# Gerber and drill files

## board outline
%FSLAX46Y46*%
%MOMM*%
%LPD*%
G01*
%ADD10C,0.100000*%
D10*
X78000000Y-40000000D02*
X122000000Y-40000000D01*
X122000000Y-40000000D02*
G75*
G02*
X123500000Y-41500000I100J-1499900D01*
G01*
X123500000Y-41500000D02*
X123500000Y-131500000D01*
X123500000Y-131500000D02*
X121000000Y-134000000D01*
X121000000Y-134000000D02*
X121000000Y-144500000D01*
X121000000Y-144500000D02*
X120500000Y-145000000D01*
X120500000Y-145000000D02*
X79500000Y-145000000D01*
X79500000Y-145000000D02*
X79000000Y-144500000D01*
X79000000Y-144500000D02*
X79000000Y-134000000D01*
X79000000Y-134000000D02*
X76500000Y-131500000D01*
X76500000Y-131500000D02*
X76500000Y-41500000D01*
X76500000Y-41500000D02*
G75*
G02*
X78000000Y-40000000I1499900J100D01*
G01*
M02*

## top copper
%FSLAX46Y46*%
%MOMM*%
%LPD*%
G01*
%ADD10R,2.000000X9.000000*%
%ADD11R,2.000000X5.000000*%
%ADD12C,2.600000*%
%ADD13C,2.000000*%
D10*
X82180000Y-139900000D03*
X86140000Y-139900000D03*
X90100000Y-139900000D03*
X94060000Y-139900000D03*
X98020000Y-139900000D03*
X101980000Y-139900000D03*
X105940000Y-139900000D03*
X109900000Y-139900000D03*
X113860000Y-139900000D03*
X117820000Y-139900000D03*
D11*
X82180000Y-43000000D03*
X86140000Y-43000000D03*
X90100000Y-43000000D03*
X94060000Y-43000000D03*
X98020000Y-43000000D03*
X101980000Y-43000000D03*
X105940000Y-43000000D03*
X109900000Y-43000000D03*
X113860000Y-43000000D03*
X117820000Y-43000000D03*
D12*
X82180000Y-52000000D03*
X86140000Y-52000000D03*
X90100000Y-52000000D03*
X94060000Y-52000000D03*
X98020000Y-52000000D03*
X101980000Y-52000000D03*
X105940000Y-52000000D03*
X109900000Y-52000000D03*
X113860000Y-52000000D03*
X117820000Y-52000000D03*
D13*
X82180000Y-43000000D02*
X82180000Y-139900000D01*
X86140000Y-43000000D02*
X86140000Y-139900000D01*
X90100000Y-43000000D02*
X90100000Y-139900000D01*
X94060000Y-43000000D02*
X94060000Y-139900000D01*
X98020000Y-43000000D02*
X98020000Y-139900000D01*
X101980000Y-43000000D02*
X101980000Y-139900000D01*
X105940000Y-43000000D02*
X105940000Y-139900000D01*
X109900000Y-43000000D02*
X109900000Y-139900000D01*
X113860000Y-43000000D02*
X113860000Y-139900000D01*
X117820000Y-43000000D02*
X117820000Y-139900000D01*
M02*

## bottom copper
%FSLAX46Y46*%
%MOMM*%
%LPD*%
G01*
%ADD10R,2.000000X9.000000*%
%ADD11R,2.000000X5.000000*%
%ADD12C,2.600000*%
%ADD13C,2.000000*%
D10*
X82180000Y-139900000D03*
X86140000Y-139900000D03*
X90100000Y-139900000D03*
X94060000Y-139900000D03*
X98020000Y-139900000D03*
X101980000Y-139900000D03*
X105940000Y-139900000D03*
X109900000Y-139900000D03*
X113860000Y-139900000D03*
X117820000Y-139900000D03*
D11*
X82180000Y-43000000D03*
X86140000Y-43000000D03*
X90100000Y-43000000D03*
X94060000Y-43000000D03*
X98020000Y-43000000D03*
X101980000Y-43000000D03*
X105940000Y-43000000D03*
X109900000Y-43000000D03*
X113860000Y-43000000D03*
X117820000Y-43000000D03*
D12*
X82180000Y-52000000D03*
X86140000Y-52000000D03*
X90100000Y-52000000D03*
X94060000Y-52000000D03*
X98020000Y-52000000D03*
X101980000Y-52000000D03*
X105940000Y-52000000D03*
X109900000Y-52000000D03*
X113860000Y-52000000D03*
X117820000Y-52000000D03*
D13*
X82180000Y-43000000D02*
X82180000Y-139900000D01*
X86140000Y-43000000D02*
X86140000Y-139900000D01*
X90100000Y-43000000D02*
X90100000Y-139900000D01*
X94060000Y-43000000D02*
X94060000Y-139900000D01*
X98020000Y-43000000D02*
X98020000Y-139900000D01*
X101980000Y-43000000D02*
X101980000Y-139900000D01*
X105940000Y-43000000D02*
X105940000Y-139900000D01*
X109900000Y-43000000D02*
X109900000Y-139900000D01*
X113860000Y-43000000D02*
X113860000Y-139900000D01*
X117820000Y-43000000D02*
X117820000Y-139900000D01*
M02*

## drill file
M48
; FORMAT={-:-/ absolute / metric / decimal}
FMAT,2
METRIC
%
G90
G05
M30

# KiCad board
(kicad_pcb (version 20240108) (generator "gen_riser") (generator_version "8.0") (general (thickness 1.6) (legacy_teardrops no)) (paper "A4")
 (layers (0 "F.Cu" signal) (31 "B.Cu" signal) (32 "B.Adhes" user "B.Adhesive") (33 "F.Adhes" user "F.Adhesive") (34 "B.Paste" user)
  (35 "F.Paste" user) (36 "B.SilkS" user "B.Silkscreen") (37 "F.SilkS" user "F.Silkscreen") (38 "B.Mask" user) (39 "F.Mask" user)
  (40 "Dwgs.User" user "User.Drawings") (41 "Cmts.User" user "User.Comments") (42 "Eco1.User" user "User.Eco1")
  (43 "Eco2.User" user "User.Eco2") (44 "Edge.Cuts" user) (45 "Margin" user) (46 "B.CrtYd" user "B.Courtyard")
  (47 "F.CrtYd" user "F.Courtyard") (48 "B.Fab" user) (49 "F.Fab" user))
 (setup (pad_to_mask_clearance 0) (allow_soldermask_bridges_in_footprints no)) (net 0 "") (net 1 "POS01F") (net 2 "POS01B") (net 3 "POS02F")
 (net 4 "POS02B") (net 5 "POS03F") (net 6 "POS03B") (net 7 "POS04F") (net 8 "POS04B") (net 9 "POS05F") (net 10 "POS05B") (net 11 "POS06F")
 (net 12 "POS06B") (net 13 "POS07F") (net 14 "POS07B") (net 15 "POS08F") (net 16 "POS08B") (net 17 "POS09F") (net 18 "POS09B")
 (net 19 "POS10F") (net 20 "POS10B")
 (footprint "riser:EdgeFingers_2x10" (layer "F.Cu") (at 100 40)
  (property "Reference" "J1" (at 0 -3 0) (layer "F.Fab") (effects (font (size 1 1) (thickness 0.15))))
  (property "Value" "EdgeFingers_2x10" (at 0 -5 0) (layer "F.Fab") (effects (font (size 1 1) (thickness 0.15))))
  (pad "1" smd rect (at -17.82 99.9) (size 2 9) (layers "F.Cu" "F.Mask") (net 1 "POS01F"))
  (pad "1B" smd rect (at -17.82 99.9) (size 2 9) (layers "B.Cu" "B.Mask") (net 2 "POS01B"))
  (pad "2" smd rect (at -13.86 99.9) (size 2 9) (layers "F.Cu" "F.Mask") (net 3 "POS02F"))
  (pad "2B" smd rect (at -13.86 99.9) (size 2 9) (layers "B.Cu" "B.Mask") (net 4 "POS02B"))
  (pad "3" smd rect (at -9.9 99.9) (size 2 9) (layers "F.Cu" "F.Mask") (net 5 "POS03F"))
  (pad "3B" smd rect (at -9.9 99.9) (size 2 9) (layers "B.Cu" "B.Mask") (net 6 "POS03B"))
  (pad "4" smd rect (at -5.94 99.9) (size 2 9) (layers "F.Cu" "F.Mask") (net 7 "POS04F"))
  (pad "4B" smd rect (at -5.94 99.9) (size 2 9) (layers "B.Cu" "B.Mask") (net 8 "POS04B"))
  (pad "5" smd rect (at -1.98 99.9) (size 2 9) (layers "F.Cu" "F.Mask") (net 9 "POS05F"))
  (pad "5B" smd rect (at -1.98 99.9) (size 2 9) (layers "B.Cu" "B.Mask") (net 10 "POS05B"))
  (pad "6" smd rect (at 1.98 99.9) (size 2 9) (layers "F.Cu" "F.Mask") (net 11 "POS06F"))
  (pad "6B" smd rect (at 1.98 99.9) (size 2 9) (layers "B.Cu" "B.Mask") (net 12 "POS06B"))
  (pad "7" smd rect (at 5.94 99.9) (size 2 9) (layers "F.Cu" "F.Mask") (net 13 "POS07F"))
  (pad "7B" smd rect (at 5.94 99.9) (size 2 9) (layers "B.Cu" "B.Mask") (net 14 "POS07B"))
  (pad "8" smd rect (at 9.9 99.9) (size 2 9) (layers "F.Cu" "F.Mask") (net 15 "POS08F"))
  (pad "8B" smd rect (at 9.9 99.9) (size 2 9) (layers "B.Cu" "B.Mask") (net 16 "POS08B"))
  (pad "9" smd rect (at 13.86 99.9) (size 2 9) (layers "F.Cu" "F.Mask") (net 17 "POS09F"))
  (pad "9B" smd rect (at 13.86 99.9) (size 2 9) (layers "B.Cu" "B.Mask") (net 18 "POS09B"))
  (pad "10" smd rect (at 17.82 99.9) (size 2 9) (layers "F.Cu" "F.Mask") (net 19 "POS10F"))
  (pad "10B" smd rect (at 17.82 99.9) (size 2 9) (layers "B.Cu" "B.Mask") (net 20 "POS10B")))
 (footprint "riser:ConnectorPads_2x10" (layer "F.Cu") (at 100 40)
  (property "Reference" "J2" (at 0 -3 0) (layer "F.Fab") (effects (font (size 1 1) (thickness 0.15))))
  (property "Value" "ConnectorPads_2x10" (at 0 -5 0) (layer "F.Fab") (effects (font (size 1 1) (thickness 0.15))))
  (pad "1" smd rect (at -17.82 3) (size 2 5) (layers "F.Cu" "F.Mask") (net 1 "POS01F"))
  (pad "1B" smd rect (at -17.82 3) (size 2 5) (layers "B.Cu" "B.Mask") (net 2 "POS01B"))
  (pad "2" smd rect (at -13.86 3) (size 2 5) (layers "F.Cu" "F.Mask") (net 3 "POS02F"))
  (pad "2B" smd rect (at -13.86 3) (size 2 5) (layers "B.Cu" "B.Mask") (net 4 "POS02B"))
  (pad "3" smd rect (at -9.9 3) (size 2 5) (layers "F.Cu" "F.Mask") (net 5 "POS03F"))
  (pad "3B" smd rect (at -9.9 3) (size 2 5) (layers "B.Cu" "B.Mask") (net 6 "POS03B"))
  (pad "4" smd rect (at -5.94 3) (size 2 5) (layers "F.Cu" "F.Mask") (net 7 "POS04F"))
  (pad "4B" smd rect (at -5.94 3) (size 2 5) (layers "B.Cu" "B.Mask") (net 8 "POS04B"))
  (pad "5" smd rect (at -1.98 3) (size 2 5) (layers "F.Cu" "F.Mask") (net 9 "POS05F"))
  (pad "5B" smd rect (at -1.98 3) (size 2 5) (layers "B.Cu" "B.Mask") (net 10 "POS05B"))
  (pad "6" smd rect (at 1.98 3) (size 2 5) (layers "F.Cu" "F.Mask") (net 11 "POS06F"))
  (pad "6B" smd rect (at 1.98 3) (size 2 5) (layers "B.Cu" "B.Mask") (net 12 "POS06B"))
  (pad "7" smd rect (at 5.94 3) (size 2 5) (layers "F.Cu" "F.Mask") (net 13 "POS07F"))
  (pad "7B" smd rect (at 5.94 3) (size 2 5) (layers "B.Cu" "B.Mask") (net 14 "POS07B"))
  (pad "8" smd rect (at 9.9 3) (size 2 5) (layers "F.Cu" "F.Mask") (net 15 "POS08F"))
  (pad "8B" smd rect (at 9.9 3) (size 2 5) (layers "B.Cu" "B.Mask") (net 16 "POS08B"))
  (pad "9" smd rect (at 13.86 3) (size 2 5) (layers "F.Cu" "F.Mask") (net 17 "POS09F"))
  (pad "9B" smd rect (at 13.86 3) (size 2 5) (layers "B.Cu" "B.Mask") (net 18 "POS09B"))
  (pad "10" smd rect (at 17.82 3) (size 2 5) (layers "F.Cu" "F.Mask") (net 19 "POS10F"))
  (pad "10B" smd rect (at 17.82 3) (size 2 5) (layers "B.Cu" "B.Mask") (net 20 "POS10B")))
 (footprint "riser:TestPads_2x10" (layer "F.Cu") (at 100 40)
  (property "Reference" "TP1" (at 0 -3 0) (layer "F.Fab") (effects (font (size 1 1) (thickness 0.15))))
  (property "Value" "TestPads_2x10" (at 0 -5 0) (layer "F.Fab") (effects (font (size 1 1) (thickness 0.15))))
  (pad "1" smd circle (at -17.82 12) (size 2.6 2.6) (layers "F.Cu" "F.Mask") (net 1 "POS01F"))
  (pad "1B" smd circle (at -17.82 12) (size 2.6 2.6) (layers "B.Cu" "B.Mask") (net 2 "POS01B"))
  (pad "2" smd circle (at -13.86 12) (size 2.6 2.6) (layers "F.Cu" "F.Mask") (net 3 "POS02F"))
  (pad "2B" smd circle (at -13.86 12) (size 2.6 2.6) (layers "B.Cu" "B.Mask") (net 4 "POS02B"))
  (pad "3" smd circle (at -9.9 12) (size 2.6 2.6) (layers "F.Cu" "F.Mask") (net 5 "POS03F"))
  (pad "3B" smd circle (at -9.9 12) (size 2.6 2.6) (layers "B.Cu" "B.Mask") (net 6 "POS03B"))
  (pad "4" smd circle (at -5.94 12) (size 2.6 2.6) (layers "F.Cu" "F.Mask") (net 7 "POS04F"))
  (pad "4B" smd circle (at -5.94 12) (size 2.6 2.6) (layers "B.Cu" "B.Mask") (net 8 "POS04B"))
  (pad "5" smd circle (at -1.98 12) (size 2.6 2.6) (layers "F.Cu" "F.Mask") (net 9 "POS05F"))
  (pad "5B" smd circle (at -1.98 12) (size 2.6 2.6) (layers "B.Cu" "B.Mask") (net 10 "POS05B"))
  (pad "6" smd circle (at 1.98 12) (size 2.6 2.6) (layers "F.Cu" "F.Mask") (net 11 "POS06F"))
  (pad "6B" smd circle (at 1.98 12) (size 2.6 2.6) (layers "B.Cu" "B.Mask") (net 12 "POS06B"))
  (pad "7" smd circle (at 5.94 12) (size 2.6 2.6) (layers "F.Cu" "F.Mask") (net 13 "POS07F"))
  (pad "7B" smd circle (at 5.94 12) (size 2.6 2.6) (layers "B.Cu" "B.Mask") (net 14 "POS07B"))
  (pad "8" smd circle (at 9.9 12) (size 2.6 2.6) (layers "F.Cu" "F.Mask") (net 15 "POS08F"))
  (pad "8B" smd circle (at 9.9 12) (size 2.6 2.6) (layers "B.Cu" "B.Mask") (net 16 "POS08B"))
  (pad "9" smd circle (at 13.86 12) (size 2.6 2.6) (layers "F.Cu" "F.Mask") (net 17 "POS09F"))
  (pad "9B" smd circle (at 13.86 12) (size 2.6 2.6) (layers "B.Cu" "B.Mask") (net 18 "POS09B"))
  (pad "10" smd circle (at 17.82 12) (size 2.6 2.6) (layers "F.Cu" "F.Mask") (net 19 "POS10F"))
  (pad "10B" smd circle (at 17.82 12) (size 2.6 2.6) (layers "B.Cu" "B.Mask") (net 20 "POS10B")))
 (segment (start 82.18 43) (end 82.18 139.9) (width 2) (layer "F.Cu") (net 1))
 (segment (start 82.18 43) (end 82.18 139.9) (width 2) (layer "B.Cu") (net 2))
 (segment (start 86.14 43) (end 86.14 139.9) (width 2) (layer "F.Cu") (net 3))
 (segment (start 86.14 43) (end 86.14 139.9) (width 2) (layer "B.Cu") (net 4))
 (segment (start 90.1 43) (end 90.1 139.9) (width 2) (layer "F.Cu") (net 5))
 (segment (start 90.1 43) (end 90.1 139.9) (width 2) (layer "B.Cu") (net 6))
 (segment (start 94.06 43) (end 94.06 139.9) (width 2) (layer "F.Cu") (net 7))
 (segment (start 94.06 43) (end 94.06 139.9) (width 2) (layer "B.Cu") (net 8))
 (segment (start 98.02 43) (end 98.02 139.9) (width 2) (layer "F.Cu") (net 9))
 (segment (start 98.02 43) (end 98.02 139.9) (width 2) (layer "B.Cu") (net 10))
 (segment (start 101.98 43) (end 101.98 139.9) (width 2) (layer "F.Cu") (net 11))
 (segment (start 101.98 43) (end 101.98 139.9) (width 2) (layer "B.Cu") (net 12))
 (segment (start 105.94 43) (end 105.94 139.9) (width 2) (layer "F.Cu") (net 13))
 (segment (start 105.94 43) (end 105.94 139.9) (width 2) (layer "B.Cu") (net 14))
 (segment (start 109.9 43) (end 109.9 139.9) (width 2) (layer "F.Cu") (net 15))
 (segment (start 109.9 43) (end 109.9 139.9) (width 2) (layer "B.Cu") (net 16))
 (segment (start 113.86 43) (end 113.86 139.9) (width 2) (layer "F.Cu") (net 17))
 (segment (start 113.86 43) (end 113.86 139.9) (width 2) (layer "B.Cu") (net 18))
 (segment (start 117.82 43) (end 117.82 139.9) (width 2) (layer "F.Cu") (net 19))
 (segment (start 117.82 43) (end 117.82 139.9) (width 2) (layer "B.Cu") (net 20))
 (gr_line (start 78 40) (end 122 40) (stroke (width 0.1) (type default)) (layer "Edge.Cuts"))
 (gr_arc (start 122 40) (mid 123.0607 40.4393) (end 123.5 41.5) (stroke (width 0.1) (type default)) (layer "Edge.Cuts"))
 (gr_line (start 123.5 41.5) (end 123.5 131.5) (stroke (width 0.1) (type default)) (layer "Edge.Cuts"))
 (gr_line (start 123.5 131.5) (end 121 134) (stroke (width 0.1) (type default)) (layer "Edge.Cuts"))
 (gr_line (start 121 134) (end 121 144.5) (stroke (width 0.1) (type default)) (layer "Edge.Cuts"))
 (gr_line (start 121 144.5) (end 120.5 145) (stroke (width 0.1) (type default)) (layer "Edge.Cuts"))
 (gr_line (start 120.5 145) (end 79.5 145) (stroke (width 0.1) (type default)) (layer "Edge.Cuts"))
 (gr_line (start 79.5 145) (end 79 144.5) (stroke (width 0.1) (type default)) (layer "Edge.Cuts"))
 (gr_line (start 79 144.5) (end 79 134) (stroke (width 0.1) (type default)) (layer "Edge.Cuts"))
 (gr_line (start 79 134) (end 76.5 131.5) (stroke (width 0.1) (type default)) (layer "Edge.Cuts"))
 (gr_line (start 76.5 131.5) (end 76.5 41.5) (stroke (width 0.1) (type default)) (layer "Edge.Cuts"))
 (gr_arc (start 76.5 41.5) (mid 76.9393 40.4393) (end 78 40) (stroke (width 0.1) (type default)) (layer "Edge.Cuts")))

